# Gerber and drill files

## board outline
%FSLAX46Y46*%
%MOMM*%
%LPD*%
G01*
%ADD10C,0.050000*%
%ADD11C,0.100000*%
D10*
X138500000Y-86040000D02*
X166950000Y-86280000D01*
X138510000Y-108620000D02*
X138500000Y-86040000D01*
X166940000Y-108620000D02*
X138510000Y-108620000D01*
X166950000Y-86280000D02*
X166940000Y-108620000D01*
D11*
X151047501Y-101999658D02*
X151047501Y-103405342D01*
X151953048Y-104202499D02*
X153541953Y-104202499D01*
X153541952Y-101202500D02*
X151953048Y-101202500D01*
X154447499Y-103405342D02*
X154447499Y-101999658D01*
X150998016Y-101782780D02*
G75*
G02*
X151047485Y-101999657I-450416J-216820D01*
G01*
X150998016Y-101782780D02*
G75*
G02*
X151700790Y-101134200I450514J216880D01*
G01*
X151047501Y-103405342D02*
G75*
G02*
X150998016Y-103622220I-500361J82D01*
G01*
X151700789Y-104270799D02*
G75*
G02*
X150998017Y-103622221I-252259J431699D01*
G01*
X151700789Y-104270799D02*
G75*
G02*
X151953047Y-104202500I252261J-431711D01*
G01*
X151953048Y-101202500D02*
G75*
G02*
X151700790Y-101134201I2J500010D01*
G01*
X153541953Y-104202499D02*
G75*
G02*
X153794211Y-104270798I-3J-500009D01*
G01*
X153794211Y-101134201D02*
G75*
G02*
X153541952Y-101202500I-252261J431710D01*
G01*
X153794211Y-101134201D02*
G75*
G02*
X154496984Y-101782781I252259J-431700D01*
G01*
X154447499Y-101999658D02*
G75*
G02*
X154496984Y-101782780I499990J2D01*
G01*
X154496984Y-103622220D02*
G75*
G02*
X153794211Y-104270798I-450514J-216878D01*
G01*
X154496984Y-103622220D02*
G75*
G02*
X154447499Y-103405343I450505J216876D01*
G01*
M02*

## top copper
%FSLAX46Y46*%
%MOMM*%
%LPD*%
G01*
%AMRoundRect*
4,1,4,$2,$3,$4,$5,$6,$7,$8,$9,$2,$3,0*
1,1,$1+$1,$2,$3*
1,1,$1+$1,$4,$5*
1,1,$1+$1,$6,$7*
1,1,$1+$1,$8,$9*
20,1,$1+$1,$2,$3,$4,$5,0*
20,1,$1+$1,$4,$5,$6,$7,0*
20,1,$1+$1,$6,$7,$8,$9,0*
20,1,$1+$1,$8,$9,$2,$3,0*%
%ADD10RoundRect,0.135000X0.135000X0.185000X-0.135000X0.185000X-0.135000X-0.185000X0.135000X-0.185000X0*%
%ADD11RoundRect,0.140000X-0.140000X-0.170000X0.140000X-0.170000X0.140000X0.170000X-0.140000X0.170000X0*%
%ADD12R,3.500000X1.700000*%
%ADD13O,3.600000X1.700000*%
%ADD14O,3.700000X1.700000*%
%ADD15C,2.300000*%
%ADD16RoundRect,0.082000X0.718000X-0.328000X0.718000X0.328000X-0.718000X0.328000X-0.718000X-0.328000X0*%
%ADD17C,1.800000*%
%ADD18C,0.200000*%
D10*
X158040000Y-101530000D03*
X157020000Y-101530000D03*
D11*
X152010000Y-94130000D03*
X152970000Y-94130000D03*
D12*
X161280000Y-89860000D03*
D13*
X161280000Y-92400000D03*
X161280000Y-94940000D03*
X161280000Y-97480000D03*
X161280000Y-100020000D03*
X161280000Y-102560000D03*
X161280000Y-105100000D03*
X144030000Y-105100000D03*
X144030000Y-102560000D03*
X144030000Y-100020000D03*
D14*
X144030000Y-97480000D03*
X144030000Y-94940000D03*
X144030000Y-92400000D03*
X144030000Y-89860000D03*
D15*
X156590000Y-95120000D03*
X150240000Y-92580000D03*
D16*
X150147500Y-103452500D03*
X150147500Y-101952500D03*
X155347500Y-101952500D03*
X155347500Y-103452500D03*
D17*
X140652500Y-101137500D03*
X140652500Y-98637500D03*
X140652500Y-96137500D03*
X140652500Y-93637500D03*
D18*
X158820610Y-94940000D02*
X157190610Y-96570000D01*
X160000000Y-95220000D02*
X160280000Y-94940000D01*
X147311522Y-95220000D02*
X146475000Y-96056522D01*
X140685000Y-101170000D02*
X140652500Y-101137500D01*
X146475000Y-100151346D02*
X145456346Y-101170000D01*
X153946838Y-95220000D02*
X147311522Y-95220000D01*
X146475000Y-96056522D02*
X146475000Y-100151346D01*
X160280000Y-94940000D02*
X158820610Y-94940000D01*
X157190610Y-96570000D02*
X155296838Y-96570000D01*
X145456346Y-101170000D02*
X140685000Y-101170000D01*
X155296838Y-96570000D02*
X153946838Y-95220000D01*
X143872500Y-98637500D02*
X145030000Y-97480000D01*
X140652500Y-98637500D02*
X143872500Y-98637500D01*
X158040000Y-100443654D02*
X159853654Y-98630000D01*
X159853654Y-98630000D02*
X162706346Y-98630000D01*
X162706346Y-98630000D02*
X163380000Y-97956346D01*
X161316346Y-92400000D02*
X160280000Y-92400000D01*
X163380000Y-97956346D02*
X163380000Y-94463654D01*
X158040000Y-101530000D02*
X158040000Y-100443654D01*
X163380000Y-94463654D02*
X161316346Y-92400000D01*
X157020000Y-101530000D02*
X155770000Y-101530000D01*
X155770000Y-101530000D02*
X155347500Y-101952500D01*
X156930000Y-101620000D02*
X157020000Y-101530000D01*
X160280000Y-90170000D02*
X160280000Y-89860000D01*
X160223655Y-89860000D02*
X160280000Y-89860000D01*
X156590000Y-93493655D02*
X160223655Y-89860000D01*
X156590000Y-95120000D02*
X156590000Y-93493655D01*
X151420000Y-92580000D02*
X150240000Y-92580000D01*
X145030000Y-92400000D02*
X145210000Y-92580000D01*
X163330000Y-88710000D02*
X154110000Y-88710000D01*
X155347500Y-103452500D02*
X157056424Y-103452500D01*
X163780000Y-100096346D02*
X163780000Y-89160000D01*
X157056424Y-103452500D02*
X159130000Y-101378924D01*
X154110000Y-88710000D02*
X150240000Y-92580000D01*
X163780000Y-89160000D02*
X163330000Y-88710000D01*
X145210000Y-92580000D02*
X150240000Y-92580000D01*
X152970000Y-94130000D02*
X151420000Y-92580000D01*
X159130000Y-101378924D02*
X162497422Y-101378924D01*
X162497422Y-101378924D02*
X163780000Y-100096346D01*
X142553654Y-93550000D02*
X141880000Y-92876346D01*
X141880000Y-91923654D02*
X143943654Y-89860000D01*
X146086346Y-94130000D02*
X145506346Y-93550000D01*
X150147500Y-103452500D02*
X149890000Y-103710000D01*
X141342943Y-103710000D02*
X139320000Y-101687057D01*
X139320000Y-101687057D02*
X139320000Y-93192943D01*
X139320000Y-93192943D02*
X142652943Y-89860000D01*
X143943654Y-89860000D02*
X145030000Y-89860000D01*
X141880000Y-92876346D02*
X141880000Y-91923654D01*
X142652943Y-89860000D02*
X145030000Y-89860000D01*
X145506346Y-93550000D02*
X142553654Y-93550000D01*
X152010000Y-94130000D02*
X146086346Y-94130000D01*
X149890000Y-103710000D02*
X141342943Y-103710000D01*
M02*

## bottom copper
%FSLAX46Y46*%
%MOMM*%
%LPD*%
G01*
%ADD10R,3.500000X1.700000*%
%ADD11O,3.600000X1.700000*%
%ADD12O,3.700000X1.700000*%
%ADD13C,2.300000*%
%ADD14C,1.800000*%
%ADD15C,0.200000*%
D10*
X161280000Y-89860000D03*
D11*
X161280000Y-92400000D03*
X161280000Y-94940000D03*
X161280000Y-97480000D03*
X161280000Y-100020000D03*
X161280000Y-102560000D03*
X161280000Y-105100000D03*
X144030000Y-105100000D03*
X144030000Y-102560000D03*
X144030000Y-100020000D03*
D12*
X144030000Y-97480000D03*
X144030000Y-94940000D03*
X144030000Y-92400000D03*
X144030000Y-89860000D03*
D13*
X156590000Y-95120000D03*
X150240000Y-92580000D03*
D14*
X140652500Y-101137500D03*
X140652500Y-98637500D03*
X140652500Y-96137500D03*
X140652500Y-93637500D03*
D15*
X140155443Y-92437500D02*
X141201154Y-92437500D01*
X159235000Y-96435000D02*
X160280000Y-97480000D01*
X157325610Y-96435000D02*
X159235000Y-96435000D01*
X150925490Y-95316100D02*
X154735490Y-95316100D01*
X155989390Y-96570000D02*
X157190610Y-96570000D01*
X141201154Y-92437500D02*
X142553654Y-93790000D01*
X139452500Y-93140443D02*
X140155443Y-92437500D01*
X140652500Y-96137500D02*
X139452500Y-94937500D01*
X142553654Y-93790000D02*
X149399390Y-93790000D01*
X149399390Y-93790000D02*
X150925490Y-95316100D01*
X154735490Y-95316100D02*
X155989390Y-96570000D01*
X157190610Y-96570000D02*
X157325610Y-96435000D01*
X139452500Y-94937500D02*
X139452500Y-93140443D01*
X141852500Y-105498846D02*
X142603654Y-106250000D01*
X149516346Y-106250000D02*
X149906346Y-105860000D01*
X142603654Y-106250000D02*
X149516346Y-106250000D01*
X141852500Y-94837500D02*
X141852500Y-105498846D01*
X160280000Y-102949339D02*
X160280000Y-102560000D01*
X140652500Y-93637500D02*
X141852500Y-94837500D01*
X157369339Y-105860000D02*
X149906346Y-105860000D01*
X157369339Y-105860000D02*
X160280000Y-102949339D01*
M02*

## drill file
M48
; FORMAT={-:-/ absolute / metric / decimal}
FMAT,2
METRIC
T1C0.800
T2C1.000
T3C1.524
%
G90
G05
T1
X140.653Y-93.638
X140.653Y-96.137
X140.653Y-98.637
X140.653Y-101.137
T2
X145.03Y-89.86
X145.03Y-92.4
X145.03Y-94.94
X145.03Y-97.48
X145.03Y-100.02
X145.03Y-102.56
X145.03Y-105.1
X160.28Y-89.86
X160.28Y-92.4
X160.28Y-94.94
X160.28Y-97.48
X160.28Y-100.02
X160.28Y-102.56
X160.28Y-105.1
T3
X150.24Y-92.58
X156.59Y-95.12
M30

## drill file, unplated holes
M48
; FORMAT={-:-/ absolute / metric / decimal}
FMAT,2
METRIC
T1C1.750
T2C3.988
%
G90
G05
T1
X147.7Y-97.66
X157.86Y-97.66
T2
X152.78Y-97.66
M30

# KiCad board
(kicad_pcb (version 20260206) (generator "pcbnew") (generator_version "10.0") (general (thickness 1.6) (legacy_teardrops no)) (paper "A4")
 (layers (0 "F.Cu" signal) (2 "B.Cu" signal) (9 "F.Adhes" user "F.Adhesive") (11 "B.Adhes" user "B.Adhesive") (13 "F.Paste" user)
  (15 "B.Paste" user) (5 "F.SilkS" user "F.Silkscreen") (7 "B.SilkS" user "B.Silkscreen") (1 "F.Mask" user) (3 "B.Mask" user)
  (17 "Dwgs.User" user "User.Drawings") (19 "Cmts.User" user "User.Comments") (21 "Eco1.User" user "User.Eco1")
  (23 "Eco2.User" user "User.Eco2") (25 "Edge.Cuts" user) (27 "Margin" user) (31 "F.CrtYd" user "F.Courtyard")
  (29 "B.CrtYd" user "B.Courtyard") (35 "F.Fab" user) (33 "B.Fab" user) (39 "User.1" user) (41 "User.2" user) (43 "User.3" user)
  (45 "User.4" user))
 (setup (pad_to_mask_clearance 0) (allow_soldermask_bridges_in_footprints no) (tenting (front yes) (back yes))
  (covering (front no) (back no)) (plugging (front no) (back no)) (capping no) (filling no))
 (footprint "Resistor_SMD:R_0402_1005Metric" (layer "F.Cu") (at 157.53 101.53 180)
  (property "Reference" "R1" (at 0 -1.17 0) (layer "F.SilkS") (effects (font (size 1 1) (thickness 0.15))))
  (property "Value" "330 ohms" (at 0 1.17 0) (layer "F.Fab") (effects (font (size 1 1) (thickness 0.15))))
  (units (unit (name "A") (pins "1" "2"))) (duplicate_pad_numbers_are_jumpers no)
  (pad "1" smd roundrect (at -0.51 0 180) (size 0.54 0.64) (layers "F.Cu" "F.Mask" "F.Paste") (roundrect_rratio 0.25) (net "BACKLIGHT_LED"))
  (pad "2" smd roundrect (at 0.51 0 180) (size 0.54 0.64) (layers "F.Cu" "F.Mask" "F.Paste") (roundrect_rratio 0.25) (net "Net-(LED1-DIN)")))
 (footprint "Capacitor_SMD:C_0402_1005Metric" (layer "F.Cu") (at 152.49 94.13)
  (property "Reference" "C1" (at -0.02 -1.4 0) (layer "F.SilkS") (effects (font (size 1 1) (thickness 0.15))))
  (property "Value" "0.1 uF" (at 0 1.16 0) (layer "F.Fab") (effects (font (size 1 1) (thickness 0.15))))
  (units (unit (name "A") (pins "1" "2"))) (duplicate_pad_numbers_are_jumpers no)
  (pad "1" smd roundrect (at -0.48 0) (size 0.56 0.62) (layers "F.Cu" "F.Mask" "F.Paste") (roundrect_rratio 0.25) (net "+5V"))
  (pad "2" smd roundrect (at 0.48 0) (size 0.56 0.62) (layers "F.Cu" "F.Mask" "F.Paste") (roundrect_rratio 0.25) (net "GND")))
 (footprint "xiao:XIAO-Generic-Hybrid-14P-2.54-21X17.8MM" (layer "B.Cu") (at 152.655 97.48 180)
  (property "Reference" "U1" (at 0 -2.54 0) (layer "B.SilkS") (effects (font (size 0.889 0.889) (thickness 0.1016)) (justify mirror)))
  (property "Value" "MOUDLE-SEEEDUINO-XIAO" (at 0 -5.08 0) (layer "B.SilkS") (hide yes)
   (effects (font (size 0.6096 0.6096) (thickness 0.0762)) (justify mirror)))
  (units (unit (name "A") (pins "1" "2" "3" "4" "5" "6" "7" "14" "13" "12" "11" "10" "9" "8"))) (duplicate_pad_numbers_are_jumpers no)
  (pad "1" thru_hole rect (at -7.625 7.62 180) (size 3.5 1.7) (drill 1 (offset -1 0)) (layers "*.Cu" "*.Mask") (remove_unused_layers no)
   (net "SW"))
  (pad "2" thru_hole oval (at -7.625 5.08 180) (size 3.6 1.7) (drill 1 (offset -1 0)) (layers "*.Cu" "*.Mask") (remove_unused_layers no)
   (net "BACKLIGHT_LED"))
  (pad "3" thru_hole oval (at -7.625 2.54 180) (size 3.6 1.7) (drill 1 (offset -1 0)) (layers "*.Cu" "*.Mask") (remove_unused_layers no)
   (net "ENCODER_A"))
  (pad "4" thru_hole oval (at -7.625 0 180) (size 3.6 1.7) (drill 1 (offset -1 0)) (layers "*.Cu" "*.Mask") (remove_unused_layers no)
   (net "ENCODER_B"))
  (pad "5" thru_hole oval (at -7.625 -2.54 180) (size 3.6 1.7) (drill 1 (offset -1 0)) (layers "*.Cu" "*.Mask") (remove_unused_layers no)
   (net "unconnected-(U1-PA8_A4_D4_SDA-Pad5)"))
  (pad "6" thru_hole oval (at -7.625 -5.08) (size 3.6 1.7) (drill 1 (offset 1 0)) (layers "*.Cu" "*.Mask") (remove_unused_layers no)
   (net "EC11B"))
  (pad "7" thru_hole oval (at -7.625 -7.62 180) (size 3.6 1.7) (drill 1 (offset -1 0)) (layers "*.Cu" "*.Mask") (remove_unused_layers no)
   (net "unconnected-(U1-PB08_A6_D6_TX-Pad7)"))
  (pad "8" thru_hole oval (at 7.625 -7.62 180) (size 3.6 1.7) (drill 1 (offset 1 0)) (layers "*.Cu" "*.Mask") (remove_unused_layers no)
   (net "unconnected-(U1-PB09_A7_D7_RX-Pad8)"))
  (pad "9" thru_hole oval (at 7.625 -5.08 180) (size 3.6 1.7) (drill 1 (offset 1 0)) (layers "*.Cu" "*.Mask") (remove_unused_layers no)
   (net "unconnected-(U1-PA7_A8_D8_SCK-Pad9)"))
  (pad "10" thru_hole oval (at 7.625 -2.54 180) (size 3.6 1.7) (drill 1 (offset 1 0)) (layers "*.Cu" "*.Mask") (remove_unused_layers no)
   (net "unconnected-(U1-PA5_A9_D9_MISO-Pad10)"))
  (pad "11" thru_hole oval (at 7.625 0 180) (size 3.7 1.7) (drill 1 (offset 1 0)) (layers "*.Cu" "*.Mask") (remove_unused_layers no)
   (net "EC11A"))
  (pad "12" thru_hole oval (at 7.625 2.54 180) (size 3.7 1.7) (drill 1 (offset 1 0)) (layers "*.Cu" "*.Mask") (remove_unused_layers no)
   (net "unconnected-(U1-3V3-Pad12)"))
  (pad "13" thru_hole oval (at 7.625 5.08 180) (size 3.7 1.7) (drill 1 (offset 1 0)) (layers "*.Cu" "*.Mask") (remove_unused_layers no)
   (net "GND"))
  (pad "14" thru_hole oval (at 7.625 7.62 180) (size 3.7 1.7) (drill 1 (offset 1 0)) (layers "*.Cu" "*.Mask") (remove_unused_layers no)
   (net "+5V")))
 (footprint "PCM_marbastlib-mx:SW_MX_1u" (layer "B.Cu") (at 152.78 97.66 180)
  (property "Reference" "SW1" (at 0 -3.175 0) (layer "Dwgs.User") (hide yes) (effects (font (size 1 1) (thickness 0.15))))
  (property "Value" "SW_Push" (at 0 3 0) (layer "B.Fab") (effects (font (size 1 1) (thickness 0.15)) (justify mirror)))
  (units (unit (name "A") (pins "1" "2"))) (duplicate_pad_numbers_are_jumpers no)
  (pad "" np_thru_hole circle (at -5.08 0 180) (size 1.75 1.75) (drill 1.75) (layers "*.Cu" "*.Mask"))
  (pad "" np_thru_hole circle (at 0 0 180) (size 3.9878 3.9878) (drill 3.9878) (layers "*.Cu" "*.Mask"))
  (pad "" np_thru_hole circle (at 5.08 0 180) (size 1.75 1.75) (drill 1.75) (layers "*.Cu" "*.Mask"))
  (pad "1" thru_hole circle (at -3.81 2.54 180) (size 2.3 2.3) (drill 1.524) (layers "*.Cu" "F.Mask") (remove_unused_layers no) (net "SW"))
  (pad "2" thru_hole circle (at 2.54 5.08 180) (size 2.3 2.3) (drill 1.524) (layers "*.Cu" "F.Mask") (remove_unused_layers no) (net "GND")))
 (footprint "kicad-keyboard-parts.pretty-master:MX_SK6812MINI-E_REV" (layer "B.Cu") (at 152.7475 97.6225 180)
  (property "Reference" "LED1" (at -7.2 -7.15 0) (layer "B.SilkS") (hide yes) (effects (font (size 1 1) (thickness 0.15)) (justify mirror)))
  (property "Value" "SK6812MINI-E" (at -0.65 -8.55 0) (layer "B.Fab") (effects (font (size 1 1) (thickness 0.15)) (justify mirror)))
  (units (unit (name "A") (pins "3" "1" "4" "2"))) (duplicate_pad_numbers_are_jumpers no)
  (fp_line (start 1.699999 -4.377158) (end 1.699999 -5.782842) (stroke (width 0.1) (type solid)) (layer "Edge.Cuts"))
  (fp_line (start 0.794452 -6.579999) (end -0.794453 -6.579999) (stroke (width 0.1) (type solid)) (layer "Edge.Cuts"))
  (fp_line (start -0.794452 -3.58) (end 0.794452 -3.58) (stroke (width 0.1) (type solid)) (layer "Edge.Cuts"))
  (fp_line (start -1.699999 -5.782842) (end -1.699999 -4.377158) (stroke (width 0.1) (type solid)) (layer "Edge.Cuts"))
  (fp_arc (start 1.749484 -4.16028) (mid 1.712526 -4.265931) (end 1.699999 -4.377157) (stroke (width 0.1) (type solid)) (layer "Edge.Cuts"))
  (fp_arc (start 1.749484 -4.16028) (mid 1.638072 -3.575963) (end 1.046711 -3.511703) (stroke (width 0.1) (type solid)) (layer "Edge.Cuts"))
  (fp_arc (start 1.699999 -5.782842) (mid 1.712536 -5.894065) (end 1.749484 -5.99972) (stroke (width 0.1) (type solid)) (layer "Edge.Cuts"))
  (fp_arc (start 1.046711 -6.648299) (mid 1.638071 -6.584036) (end 1.749484 -5.99972) (stroke (width 0.1) (type solid)) (layer "Edge.Cuts"))
  (fp_arc (start 1.046711 -6.648299) (mid 0.925123 -6.597377) (end 0.794453 -6.58) (stroke (width 0.1) (type solid)) (layer "Edge.Cuts"))
  (fp_arc (start 0.794452 -3.58) (mid 0.925122 -3.562623) (end 1.04671 -3.511701) (stroke (width 0.1) (type solid)) (layer "Edge.Cuts"))
  (fp_arc (start -0.794453 -6.579999) (mid -0.925123 -6.597376) (end -1.046711 -6.648298) (stroke (width 0.1) (type solid))
   (layer "Edge.Cuts"))
  (fp_arc (start -1.046711 -3.511701) (mid -0.925123 -3.562623) (end -0.794452 -3.58) (stroke (width 0.1) (type solid)) (layer "Edge.Cuts"))
  (fp_arc (start -1.046711 -3.511701) (mid -1.638072 -3.575965) (end -1.749484 -4.160281) (stroke (width 0.1) (type solid))
   (layer "Edge.Cuts"))
  (fp_arc (start -1.699999 -4.377158) (mid -1.712527 -4.265932) (end -1.749484 -4.16028) (stroke (width 0.1) (type solid))
   (layer "Edge.Cuts"))
  (fp_arc (start -1.749484 -5.99972) (mid -1.638071 -6.584035) (end -1.046711 -6.648298) (stroke (width 0.1) (type solid))
   (layer "Edge.Cuts"))
  (fp_arc (start -1.749484 -5.99972) (mid -1.712527 -5.894068) (end -1.699999 -5.782843) (stroke (width 0.1) (type solid))
   (layer "Edge.Cuts"))
  (pad "1" smd roundrect (at 2.6 -5.83 90) (size 0.82 1.6) (layers "F.Cu" "F.Mask" "F.Paste") (roundrect_rratio 0.1) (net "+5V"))
  (pad "2" smd roundrect (at 2.6 -4.33 90) (size 0.82 1.6) (layers "F.Cu" "F.Mask" "F.Paste") (roundrect_rratio 0.1)
   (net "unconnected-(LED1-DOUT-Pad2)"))
  (pad "3" smd roundrect (at -2.6 -4.33 90) (size 0.82 1.6) (layers "F.Cu" "F.Mask" "F.Paste") (roundrect_rratio 0.1) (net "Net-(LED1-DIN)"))
  (pad "4" smd roundrect (at -2.6 -5.83 90) (size 0.82 1.6) (layers "F.Cu" "F.Mask" "F.Paste") (roundrect_rratio 0.1) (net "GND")))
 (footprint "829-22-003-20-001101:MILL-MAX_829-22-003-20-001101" (layer "B.Cu") (at 137.4525 108.9875)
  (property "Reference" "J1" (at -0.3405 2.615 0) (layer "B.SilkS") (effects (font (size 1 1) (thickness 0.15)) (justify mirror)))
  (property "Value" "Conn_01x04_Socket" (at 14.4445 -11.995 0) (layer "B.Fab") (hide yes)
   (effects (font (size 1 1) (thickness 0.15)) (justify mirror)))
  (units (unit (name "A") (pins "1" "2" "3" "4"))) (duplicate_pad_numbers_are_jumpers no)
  (pad "1" thru_hole circle (at 3.2 -7.85 90) (size 1.8 1.8) (drill 0.8) (layers "*.Cu" "*.Mask") (remove_unused_layers no)
   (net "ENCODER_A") (solder_mask_margin 0.102))
  (pad "2" thru_hole circle (at 3.2 -10.35 90) (size 1.8 1.8) (drill 0.8) (layers "*.Cu" "*.Mask") (remove_unused_layers no) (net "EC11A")
   (solder_mask_margin 0.102))
  (pad "3" thru_hole circle (at 3.2 -12.85 90) (size 1.8 1.8) (drill 0.8) (layers "*.Cu" "*.Mask") (remove_unused_layers no)
   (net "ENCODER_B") (solder_mask_margin 0.102))
  (pad "4" thru_hole circle (at 3.2 -15.35 90) (size 1.8 1.8) (drill 0.8) (layers "*.Cu" "*.Mask") (remove_unused_layers no) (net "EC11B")
   (solder_mask_margin 0.102)))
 (gr_line (start 138.5 86.04) (end 166.95 86.28) (stroke (width 0.05) (type default)) (layer "Edge.Cuts"))
 (gr_line (start 138.51 108.62) (end 138.5 86.04) (stroke (width 0.05) (type default)) (layer "Edge.Cuts"))
 (gr_line (start 166.94 108.62) (end 138.51 108.62) (stroke (width 0.05) (type default)) (layer "Edge.Cuts"))
 (gr_line (start 166.95 86.28) (end 166.94 108.62) (stroke (width 0.05) (type default)) (layer "Edge.Cuts"))
 (segment (start 158.82061 94.94) (end 157.19061 96.57) (width 0.2) (layer "F.Cu") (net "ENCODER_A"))
 (segment (start 160 95.22) (end 160.28 94.94) (width 0.2) (layer "F.Cu") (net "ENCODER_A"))
 (segment (start 147.311522 95.22) (end 146.475 96.056522) (width 0.2) (layer "F.Cu") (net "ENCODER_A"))
 (segment (start 140.685 101.17) (end 140.6525 101.1375) (width 0.2) (layer "F.Cu") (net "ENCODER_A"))
 (segment (start 146.475 100.151346) (end 145.456346 101.17) (width 0.2) (layer "F.Cu") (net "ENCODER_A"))
 (segment (start 153.946838 95.22) (end 147.311522 95.22) (width 0.2) (layer "F.Cu") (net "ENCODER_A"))
 (segment (start 146.475 96.056522) (end 146.475 100.151346) (width 0.2) (layer "F.Cu") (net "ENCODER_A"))
 (segment (start 160.28 94.94) (end 158.82061 94.94) (width 0.2) (layer "F.Cu") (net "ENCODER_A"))
 (segment (start 157.19061 96.57) (end 155.296838 96.57) (width 0.2) (layer "F.Cu") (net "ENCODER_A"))
 (segment (start 145.456346 101.17) (end 140.685 101.17) (width 0.2) (layer "F.Cu") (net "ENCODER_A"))
 (segment (start 155.296838 96.57) (end 153.946838 95.22) (width 0.2) (layer "F.Cu") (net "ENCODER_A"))
 (segment (start 143.8725 98.6375) (end 145.03 97.48) (width 0.2) (layer "F.Cu") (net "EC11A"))
 (segment (start 140.6525 98.6375) (end 143.8725 98.6375) (width 0.2) (layer "F.Cu") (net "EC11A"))
 (segment (start 140.155443 92.4375) (end 141.201154 92.4375) (width 0.2) (layer "B.Cu") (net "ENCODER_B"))
 (segment (start 159.235 96.435) (end 160.28 97.48) (width 0.2) (layer "B.Cu") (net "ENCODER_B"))
 (segment (start 157.32561 96.435) (end 159.235 96.435) (width 0.2) (layer "B.Cu") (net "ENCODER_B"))
 (segment (start 150.92549 95.3161) (end 154.73549 95.3161) (width 0.2) (layer "B.Cu") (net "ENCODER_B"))
 (segment (start 155.98939 96.57) (end 157.19061 96.57) (width 0.2) (layer "B.Cu") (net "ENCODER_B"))
 (segment (start 141.201154 92.4375) (end 142.553654 93.79) (width 0.2) (layer "B.Cu") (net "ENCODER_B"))
 (segment (start 139.4525 93.140443) (end 140.155443 92.4375) (width 0.2) (layer "B.Cu") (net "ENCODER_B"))
 (segment (start 140.6525 96.1375) (end 139.4525 94.9375) (width 0.2) (layer "B.Cu") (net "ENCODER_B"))
 (segment (start 142.553654 93.79) (end 149.39939 93.79) (width 0.2) (layer "B.Cu") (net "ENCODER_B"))
 (segment (start 149.39939 93.79) (end 150.92549 95.3161) (width 0.2) (layer "B.Cu") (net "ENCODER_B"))
 (segment (start 154.73549 95.3161) (end 155.98939 96.57) (width 0.2) (layer "B.Cu") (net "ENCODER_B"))
 (segment (start 157.19061 96.57) (end 157.32561 96.435) (width 0.2) (layer "B.Cu") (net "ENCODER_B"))
 (segment (start 139.4525 94.9375) (end 139.4525 93.140443) (width 0.2) (layer "B.Cu") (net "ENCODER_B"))
 (segment (start 141.8525 105.498846) (end 142.603654 106.25) (width 0.2) (layer "B.Cu") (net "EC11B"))
 (segment (start 149.516346 106.25) (end 149.906346 105.86) (width 0.2) (layer "B.Cu") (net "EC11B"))
 (segment (start 142.603654 106.25) (end 149.516346 106.25) (width 0.2) (layer "B.Cu") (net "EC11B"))
 (segment (start 141.8525 94.8375) (end 141.8525 105.498846) (width 0.2) (layer "B.Cu") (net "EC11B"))
 (segment (start 160.28 102.949339) (end 160.28 102.56) (width 0.2) (layer "B.Cu") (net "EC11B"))
 (segment (start 140.6525 93.6375) (end 141.8525 94.8375) (width 0.2) (layer "B.Cu") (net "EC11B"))
 (segment (start 157.369339 105.86) (end 149.906346 105.86) (width 0.2) (layer "B.Cu") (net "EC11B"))
 (segment (start 157.369339 105.86) (end 160.28 102.949339) (width 0.2) (layer "B.Cu") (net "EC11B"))
 (segment (start 158.04 100.443654) (end 159.853654 98.63) (width 0.2) (layer "F.Cu") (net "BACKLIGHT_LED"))
 (segment (start 159.853654 98.63) (end 162.706346 98.63) (width 0.2) (layer "F.Cu") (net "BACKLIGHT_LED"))
 (segment (start 162.706346 98.63) (end 163.38 97.956346) (width 0.2) (layer "F.Cu") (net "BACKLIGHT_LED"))
 (segment (start 161.316346 92.4) (end 160.28 92.4) (width 0.2) (layer "F.Cu") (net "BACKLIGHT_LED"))
 (segment (start 163.38 97.956346) (end 163.38 94.463654) (width 0.2) (layer "F.Cu") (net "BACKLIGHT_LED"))
 (segment (start 158.04 101.53) (end 158.04 100.443654) (width 0.2) (layer "F.Cu") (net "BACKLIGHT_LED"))
 (segment (start 163.38 94.463654) (end 161.316346 92.4) (width 0.2) (layer "F.Cu") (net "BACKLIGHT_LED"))
 (segment (start 157.02 101.53) (end 155.77 101.53) (width 0.2) (layer "F.Cu") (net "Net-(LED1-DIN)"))
 (segment (start 155.77 101.53) (end 155.3475 101.9525) (width 0.2) (layer "F.Cu") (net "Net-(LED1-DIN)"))
 (segment (start 156.93 101.62) (end 157.02 101.53) (width 0.2) (layer "F.Cu") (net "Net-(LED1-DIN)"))
 (segment (start 160.28 90.17) (end 160.28 89.86) (width 0.2) (layer "F.Cu") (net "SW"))
 (segment (start 160.223655 89.86) (end 160.28 89.86) (width 0.2) (layer "F.Cu") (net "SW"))
 (segment (start 156.59 93.493655) (end 160.223655 89.86) (width 0.2) (layer "F.Cu") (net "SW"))
 (segment (start 156.59 95.12) (end 156.59 93.493655) (width 0.2) (layer "F.Cu") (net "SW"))
 (segment (start 151.42 92.58) (end 150.24 92.58) (width 0.2) (layer "F.Cu") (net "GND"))
 (segment (start 145.03 92.4) (end 145.21 92.58) (width 0.2) (layer "F.Cu") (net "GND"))
 (segment (start 163.33 88.71) (end 154.11 88.71) (width 0.2) (layer "F.Cu") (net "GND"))
 (segment (start 155.3475 103.4525) (end 157.056424 103.4525) (width 0.2) (layer "F.Cu") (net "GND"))
 (segment (start 163.78 100.096346) (end 163.78 89.16) (width 0.2) (layer "F.Cu") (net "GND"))
 (segment (start 157.056424 103.4525) (end 159.13 101.378924) (width 0.2) (layer "F.Cu") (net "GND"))
 (segment (start 154.11 88.71) (end 150.24 92.58) (width 0.2) (layer "F.Cu") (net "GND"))
 (segment (start 163.78 89.16) (end 163.33 88.71) (width 0.2) (layer "F.Cu") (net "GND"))
 (segment (start 145.21 92.58) (end 150.24 92.58) (width 0.2) (layer "F.Cu") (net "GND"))
 (segment (start 152.97 94.13) (end 151.42 92.58) (width 0.2) (layer "F.Cu") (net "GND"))
 (segment (start 159.13 101.378924) (end 162.497422 101.378924) (width 0.2) (layer "F.Cu") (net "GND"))
 (segment (start 162.497422 101.378924) (end 163.78 100.096346) (width 0.2) (layer "F.Cu") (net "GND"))
 (segment (start 142.553654 93.55) (end 141.88 92.876346) (width 0.2) (layer "F.Cu") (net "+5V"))
 (segment (start 141.88 91.923654) (end 143.943654 89.86) (width 0.2) (layer "F.Cu") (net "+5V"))
 (segment (start 146.086346 94.13) (end 145.506346 93.55) (width 0.2) (layer "F.Cu") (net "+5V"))
 (segment (start 150.1475 103.4525) (end 149.89 103.71) (width 0.2) (layer "F.Cu") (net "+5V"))
 (segment (start 141.342943 103.71) (end 139.32 101.687057) (width 0.2) (layer "F.Cu") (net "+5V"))
 (segment (start 139.32 101.687057) (end 139.32 93.192943) (width 0.2) (layer "F.Cu") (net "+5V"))
 (segment (start 139.32 93.192943) (end 142.652943 89.86) (width 0.2) (layer "F.Cu") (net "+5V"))
 (segment (start 143.943654 89.86) (end 145.03 89.86) (width 0.2) (layer "F.Cu") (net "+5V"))
 (segment (start 141.88 92.876346) (end 141.88 91.923654) (width 0.2) (layer "F.Cu") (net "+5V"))
 (segment (start 142.652943 89.86) (end 145.03 89.86) (width 0.2) (layer "F.Cu") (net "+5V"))
 (segment (start 145.506346 93.55) (end 142.553654 93.55) (width 0.2) (layer "F.Cu") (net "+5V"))
 (segment (start 152.01 94.13) (end 146.086346 94.13) (width 0.2) (layer "F.Cu") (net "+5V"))
 (segment (start 149.89 103.71) (end 141.342943 103.71) (width 0.2) (layer "F.Cu") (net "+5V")))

